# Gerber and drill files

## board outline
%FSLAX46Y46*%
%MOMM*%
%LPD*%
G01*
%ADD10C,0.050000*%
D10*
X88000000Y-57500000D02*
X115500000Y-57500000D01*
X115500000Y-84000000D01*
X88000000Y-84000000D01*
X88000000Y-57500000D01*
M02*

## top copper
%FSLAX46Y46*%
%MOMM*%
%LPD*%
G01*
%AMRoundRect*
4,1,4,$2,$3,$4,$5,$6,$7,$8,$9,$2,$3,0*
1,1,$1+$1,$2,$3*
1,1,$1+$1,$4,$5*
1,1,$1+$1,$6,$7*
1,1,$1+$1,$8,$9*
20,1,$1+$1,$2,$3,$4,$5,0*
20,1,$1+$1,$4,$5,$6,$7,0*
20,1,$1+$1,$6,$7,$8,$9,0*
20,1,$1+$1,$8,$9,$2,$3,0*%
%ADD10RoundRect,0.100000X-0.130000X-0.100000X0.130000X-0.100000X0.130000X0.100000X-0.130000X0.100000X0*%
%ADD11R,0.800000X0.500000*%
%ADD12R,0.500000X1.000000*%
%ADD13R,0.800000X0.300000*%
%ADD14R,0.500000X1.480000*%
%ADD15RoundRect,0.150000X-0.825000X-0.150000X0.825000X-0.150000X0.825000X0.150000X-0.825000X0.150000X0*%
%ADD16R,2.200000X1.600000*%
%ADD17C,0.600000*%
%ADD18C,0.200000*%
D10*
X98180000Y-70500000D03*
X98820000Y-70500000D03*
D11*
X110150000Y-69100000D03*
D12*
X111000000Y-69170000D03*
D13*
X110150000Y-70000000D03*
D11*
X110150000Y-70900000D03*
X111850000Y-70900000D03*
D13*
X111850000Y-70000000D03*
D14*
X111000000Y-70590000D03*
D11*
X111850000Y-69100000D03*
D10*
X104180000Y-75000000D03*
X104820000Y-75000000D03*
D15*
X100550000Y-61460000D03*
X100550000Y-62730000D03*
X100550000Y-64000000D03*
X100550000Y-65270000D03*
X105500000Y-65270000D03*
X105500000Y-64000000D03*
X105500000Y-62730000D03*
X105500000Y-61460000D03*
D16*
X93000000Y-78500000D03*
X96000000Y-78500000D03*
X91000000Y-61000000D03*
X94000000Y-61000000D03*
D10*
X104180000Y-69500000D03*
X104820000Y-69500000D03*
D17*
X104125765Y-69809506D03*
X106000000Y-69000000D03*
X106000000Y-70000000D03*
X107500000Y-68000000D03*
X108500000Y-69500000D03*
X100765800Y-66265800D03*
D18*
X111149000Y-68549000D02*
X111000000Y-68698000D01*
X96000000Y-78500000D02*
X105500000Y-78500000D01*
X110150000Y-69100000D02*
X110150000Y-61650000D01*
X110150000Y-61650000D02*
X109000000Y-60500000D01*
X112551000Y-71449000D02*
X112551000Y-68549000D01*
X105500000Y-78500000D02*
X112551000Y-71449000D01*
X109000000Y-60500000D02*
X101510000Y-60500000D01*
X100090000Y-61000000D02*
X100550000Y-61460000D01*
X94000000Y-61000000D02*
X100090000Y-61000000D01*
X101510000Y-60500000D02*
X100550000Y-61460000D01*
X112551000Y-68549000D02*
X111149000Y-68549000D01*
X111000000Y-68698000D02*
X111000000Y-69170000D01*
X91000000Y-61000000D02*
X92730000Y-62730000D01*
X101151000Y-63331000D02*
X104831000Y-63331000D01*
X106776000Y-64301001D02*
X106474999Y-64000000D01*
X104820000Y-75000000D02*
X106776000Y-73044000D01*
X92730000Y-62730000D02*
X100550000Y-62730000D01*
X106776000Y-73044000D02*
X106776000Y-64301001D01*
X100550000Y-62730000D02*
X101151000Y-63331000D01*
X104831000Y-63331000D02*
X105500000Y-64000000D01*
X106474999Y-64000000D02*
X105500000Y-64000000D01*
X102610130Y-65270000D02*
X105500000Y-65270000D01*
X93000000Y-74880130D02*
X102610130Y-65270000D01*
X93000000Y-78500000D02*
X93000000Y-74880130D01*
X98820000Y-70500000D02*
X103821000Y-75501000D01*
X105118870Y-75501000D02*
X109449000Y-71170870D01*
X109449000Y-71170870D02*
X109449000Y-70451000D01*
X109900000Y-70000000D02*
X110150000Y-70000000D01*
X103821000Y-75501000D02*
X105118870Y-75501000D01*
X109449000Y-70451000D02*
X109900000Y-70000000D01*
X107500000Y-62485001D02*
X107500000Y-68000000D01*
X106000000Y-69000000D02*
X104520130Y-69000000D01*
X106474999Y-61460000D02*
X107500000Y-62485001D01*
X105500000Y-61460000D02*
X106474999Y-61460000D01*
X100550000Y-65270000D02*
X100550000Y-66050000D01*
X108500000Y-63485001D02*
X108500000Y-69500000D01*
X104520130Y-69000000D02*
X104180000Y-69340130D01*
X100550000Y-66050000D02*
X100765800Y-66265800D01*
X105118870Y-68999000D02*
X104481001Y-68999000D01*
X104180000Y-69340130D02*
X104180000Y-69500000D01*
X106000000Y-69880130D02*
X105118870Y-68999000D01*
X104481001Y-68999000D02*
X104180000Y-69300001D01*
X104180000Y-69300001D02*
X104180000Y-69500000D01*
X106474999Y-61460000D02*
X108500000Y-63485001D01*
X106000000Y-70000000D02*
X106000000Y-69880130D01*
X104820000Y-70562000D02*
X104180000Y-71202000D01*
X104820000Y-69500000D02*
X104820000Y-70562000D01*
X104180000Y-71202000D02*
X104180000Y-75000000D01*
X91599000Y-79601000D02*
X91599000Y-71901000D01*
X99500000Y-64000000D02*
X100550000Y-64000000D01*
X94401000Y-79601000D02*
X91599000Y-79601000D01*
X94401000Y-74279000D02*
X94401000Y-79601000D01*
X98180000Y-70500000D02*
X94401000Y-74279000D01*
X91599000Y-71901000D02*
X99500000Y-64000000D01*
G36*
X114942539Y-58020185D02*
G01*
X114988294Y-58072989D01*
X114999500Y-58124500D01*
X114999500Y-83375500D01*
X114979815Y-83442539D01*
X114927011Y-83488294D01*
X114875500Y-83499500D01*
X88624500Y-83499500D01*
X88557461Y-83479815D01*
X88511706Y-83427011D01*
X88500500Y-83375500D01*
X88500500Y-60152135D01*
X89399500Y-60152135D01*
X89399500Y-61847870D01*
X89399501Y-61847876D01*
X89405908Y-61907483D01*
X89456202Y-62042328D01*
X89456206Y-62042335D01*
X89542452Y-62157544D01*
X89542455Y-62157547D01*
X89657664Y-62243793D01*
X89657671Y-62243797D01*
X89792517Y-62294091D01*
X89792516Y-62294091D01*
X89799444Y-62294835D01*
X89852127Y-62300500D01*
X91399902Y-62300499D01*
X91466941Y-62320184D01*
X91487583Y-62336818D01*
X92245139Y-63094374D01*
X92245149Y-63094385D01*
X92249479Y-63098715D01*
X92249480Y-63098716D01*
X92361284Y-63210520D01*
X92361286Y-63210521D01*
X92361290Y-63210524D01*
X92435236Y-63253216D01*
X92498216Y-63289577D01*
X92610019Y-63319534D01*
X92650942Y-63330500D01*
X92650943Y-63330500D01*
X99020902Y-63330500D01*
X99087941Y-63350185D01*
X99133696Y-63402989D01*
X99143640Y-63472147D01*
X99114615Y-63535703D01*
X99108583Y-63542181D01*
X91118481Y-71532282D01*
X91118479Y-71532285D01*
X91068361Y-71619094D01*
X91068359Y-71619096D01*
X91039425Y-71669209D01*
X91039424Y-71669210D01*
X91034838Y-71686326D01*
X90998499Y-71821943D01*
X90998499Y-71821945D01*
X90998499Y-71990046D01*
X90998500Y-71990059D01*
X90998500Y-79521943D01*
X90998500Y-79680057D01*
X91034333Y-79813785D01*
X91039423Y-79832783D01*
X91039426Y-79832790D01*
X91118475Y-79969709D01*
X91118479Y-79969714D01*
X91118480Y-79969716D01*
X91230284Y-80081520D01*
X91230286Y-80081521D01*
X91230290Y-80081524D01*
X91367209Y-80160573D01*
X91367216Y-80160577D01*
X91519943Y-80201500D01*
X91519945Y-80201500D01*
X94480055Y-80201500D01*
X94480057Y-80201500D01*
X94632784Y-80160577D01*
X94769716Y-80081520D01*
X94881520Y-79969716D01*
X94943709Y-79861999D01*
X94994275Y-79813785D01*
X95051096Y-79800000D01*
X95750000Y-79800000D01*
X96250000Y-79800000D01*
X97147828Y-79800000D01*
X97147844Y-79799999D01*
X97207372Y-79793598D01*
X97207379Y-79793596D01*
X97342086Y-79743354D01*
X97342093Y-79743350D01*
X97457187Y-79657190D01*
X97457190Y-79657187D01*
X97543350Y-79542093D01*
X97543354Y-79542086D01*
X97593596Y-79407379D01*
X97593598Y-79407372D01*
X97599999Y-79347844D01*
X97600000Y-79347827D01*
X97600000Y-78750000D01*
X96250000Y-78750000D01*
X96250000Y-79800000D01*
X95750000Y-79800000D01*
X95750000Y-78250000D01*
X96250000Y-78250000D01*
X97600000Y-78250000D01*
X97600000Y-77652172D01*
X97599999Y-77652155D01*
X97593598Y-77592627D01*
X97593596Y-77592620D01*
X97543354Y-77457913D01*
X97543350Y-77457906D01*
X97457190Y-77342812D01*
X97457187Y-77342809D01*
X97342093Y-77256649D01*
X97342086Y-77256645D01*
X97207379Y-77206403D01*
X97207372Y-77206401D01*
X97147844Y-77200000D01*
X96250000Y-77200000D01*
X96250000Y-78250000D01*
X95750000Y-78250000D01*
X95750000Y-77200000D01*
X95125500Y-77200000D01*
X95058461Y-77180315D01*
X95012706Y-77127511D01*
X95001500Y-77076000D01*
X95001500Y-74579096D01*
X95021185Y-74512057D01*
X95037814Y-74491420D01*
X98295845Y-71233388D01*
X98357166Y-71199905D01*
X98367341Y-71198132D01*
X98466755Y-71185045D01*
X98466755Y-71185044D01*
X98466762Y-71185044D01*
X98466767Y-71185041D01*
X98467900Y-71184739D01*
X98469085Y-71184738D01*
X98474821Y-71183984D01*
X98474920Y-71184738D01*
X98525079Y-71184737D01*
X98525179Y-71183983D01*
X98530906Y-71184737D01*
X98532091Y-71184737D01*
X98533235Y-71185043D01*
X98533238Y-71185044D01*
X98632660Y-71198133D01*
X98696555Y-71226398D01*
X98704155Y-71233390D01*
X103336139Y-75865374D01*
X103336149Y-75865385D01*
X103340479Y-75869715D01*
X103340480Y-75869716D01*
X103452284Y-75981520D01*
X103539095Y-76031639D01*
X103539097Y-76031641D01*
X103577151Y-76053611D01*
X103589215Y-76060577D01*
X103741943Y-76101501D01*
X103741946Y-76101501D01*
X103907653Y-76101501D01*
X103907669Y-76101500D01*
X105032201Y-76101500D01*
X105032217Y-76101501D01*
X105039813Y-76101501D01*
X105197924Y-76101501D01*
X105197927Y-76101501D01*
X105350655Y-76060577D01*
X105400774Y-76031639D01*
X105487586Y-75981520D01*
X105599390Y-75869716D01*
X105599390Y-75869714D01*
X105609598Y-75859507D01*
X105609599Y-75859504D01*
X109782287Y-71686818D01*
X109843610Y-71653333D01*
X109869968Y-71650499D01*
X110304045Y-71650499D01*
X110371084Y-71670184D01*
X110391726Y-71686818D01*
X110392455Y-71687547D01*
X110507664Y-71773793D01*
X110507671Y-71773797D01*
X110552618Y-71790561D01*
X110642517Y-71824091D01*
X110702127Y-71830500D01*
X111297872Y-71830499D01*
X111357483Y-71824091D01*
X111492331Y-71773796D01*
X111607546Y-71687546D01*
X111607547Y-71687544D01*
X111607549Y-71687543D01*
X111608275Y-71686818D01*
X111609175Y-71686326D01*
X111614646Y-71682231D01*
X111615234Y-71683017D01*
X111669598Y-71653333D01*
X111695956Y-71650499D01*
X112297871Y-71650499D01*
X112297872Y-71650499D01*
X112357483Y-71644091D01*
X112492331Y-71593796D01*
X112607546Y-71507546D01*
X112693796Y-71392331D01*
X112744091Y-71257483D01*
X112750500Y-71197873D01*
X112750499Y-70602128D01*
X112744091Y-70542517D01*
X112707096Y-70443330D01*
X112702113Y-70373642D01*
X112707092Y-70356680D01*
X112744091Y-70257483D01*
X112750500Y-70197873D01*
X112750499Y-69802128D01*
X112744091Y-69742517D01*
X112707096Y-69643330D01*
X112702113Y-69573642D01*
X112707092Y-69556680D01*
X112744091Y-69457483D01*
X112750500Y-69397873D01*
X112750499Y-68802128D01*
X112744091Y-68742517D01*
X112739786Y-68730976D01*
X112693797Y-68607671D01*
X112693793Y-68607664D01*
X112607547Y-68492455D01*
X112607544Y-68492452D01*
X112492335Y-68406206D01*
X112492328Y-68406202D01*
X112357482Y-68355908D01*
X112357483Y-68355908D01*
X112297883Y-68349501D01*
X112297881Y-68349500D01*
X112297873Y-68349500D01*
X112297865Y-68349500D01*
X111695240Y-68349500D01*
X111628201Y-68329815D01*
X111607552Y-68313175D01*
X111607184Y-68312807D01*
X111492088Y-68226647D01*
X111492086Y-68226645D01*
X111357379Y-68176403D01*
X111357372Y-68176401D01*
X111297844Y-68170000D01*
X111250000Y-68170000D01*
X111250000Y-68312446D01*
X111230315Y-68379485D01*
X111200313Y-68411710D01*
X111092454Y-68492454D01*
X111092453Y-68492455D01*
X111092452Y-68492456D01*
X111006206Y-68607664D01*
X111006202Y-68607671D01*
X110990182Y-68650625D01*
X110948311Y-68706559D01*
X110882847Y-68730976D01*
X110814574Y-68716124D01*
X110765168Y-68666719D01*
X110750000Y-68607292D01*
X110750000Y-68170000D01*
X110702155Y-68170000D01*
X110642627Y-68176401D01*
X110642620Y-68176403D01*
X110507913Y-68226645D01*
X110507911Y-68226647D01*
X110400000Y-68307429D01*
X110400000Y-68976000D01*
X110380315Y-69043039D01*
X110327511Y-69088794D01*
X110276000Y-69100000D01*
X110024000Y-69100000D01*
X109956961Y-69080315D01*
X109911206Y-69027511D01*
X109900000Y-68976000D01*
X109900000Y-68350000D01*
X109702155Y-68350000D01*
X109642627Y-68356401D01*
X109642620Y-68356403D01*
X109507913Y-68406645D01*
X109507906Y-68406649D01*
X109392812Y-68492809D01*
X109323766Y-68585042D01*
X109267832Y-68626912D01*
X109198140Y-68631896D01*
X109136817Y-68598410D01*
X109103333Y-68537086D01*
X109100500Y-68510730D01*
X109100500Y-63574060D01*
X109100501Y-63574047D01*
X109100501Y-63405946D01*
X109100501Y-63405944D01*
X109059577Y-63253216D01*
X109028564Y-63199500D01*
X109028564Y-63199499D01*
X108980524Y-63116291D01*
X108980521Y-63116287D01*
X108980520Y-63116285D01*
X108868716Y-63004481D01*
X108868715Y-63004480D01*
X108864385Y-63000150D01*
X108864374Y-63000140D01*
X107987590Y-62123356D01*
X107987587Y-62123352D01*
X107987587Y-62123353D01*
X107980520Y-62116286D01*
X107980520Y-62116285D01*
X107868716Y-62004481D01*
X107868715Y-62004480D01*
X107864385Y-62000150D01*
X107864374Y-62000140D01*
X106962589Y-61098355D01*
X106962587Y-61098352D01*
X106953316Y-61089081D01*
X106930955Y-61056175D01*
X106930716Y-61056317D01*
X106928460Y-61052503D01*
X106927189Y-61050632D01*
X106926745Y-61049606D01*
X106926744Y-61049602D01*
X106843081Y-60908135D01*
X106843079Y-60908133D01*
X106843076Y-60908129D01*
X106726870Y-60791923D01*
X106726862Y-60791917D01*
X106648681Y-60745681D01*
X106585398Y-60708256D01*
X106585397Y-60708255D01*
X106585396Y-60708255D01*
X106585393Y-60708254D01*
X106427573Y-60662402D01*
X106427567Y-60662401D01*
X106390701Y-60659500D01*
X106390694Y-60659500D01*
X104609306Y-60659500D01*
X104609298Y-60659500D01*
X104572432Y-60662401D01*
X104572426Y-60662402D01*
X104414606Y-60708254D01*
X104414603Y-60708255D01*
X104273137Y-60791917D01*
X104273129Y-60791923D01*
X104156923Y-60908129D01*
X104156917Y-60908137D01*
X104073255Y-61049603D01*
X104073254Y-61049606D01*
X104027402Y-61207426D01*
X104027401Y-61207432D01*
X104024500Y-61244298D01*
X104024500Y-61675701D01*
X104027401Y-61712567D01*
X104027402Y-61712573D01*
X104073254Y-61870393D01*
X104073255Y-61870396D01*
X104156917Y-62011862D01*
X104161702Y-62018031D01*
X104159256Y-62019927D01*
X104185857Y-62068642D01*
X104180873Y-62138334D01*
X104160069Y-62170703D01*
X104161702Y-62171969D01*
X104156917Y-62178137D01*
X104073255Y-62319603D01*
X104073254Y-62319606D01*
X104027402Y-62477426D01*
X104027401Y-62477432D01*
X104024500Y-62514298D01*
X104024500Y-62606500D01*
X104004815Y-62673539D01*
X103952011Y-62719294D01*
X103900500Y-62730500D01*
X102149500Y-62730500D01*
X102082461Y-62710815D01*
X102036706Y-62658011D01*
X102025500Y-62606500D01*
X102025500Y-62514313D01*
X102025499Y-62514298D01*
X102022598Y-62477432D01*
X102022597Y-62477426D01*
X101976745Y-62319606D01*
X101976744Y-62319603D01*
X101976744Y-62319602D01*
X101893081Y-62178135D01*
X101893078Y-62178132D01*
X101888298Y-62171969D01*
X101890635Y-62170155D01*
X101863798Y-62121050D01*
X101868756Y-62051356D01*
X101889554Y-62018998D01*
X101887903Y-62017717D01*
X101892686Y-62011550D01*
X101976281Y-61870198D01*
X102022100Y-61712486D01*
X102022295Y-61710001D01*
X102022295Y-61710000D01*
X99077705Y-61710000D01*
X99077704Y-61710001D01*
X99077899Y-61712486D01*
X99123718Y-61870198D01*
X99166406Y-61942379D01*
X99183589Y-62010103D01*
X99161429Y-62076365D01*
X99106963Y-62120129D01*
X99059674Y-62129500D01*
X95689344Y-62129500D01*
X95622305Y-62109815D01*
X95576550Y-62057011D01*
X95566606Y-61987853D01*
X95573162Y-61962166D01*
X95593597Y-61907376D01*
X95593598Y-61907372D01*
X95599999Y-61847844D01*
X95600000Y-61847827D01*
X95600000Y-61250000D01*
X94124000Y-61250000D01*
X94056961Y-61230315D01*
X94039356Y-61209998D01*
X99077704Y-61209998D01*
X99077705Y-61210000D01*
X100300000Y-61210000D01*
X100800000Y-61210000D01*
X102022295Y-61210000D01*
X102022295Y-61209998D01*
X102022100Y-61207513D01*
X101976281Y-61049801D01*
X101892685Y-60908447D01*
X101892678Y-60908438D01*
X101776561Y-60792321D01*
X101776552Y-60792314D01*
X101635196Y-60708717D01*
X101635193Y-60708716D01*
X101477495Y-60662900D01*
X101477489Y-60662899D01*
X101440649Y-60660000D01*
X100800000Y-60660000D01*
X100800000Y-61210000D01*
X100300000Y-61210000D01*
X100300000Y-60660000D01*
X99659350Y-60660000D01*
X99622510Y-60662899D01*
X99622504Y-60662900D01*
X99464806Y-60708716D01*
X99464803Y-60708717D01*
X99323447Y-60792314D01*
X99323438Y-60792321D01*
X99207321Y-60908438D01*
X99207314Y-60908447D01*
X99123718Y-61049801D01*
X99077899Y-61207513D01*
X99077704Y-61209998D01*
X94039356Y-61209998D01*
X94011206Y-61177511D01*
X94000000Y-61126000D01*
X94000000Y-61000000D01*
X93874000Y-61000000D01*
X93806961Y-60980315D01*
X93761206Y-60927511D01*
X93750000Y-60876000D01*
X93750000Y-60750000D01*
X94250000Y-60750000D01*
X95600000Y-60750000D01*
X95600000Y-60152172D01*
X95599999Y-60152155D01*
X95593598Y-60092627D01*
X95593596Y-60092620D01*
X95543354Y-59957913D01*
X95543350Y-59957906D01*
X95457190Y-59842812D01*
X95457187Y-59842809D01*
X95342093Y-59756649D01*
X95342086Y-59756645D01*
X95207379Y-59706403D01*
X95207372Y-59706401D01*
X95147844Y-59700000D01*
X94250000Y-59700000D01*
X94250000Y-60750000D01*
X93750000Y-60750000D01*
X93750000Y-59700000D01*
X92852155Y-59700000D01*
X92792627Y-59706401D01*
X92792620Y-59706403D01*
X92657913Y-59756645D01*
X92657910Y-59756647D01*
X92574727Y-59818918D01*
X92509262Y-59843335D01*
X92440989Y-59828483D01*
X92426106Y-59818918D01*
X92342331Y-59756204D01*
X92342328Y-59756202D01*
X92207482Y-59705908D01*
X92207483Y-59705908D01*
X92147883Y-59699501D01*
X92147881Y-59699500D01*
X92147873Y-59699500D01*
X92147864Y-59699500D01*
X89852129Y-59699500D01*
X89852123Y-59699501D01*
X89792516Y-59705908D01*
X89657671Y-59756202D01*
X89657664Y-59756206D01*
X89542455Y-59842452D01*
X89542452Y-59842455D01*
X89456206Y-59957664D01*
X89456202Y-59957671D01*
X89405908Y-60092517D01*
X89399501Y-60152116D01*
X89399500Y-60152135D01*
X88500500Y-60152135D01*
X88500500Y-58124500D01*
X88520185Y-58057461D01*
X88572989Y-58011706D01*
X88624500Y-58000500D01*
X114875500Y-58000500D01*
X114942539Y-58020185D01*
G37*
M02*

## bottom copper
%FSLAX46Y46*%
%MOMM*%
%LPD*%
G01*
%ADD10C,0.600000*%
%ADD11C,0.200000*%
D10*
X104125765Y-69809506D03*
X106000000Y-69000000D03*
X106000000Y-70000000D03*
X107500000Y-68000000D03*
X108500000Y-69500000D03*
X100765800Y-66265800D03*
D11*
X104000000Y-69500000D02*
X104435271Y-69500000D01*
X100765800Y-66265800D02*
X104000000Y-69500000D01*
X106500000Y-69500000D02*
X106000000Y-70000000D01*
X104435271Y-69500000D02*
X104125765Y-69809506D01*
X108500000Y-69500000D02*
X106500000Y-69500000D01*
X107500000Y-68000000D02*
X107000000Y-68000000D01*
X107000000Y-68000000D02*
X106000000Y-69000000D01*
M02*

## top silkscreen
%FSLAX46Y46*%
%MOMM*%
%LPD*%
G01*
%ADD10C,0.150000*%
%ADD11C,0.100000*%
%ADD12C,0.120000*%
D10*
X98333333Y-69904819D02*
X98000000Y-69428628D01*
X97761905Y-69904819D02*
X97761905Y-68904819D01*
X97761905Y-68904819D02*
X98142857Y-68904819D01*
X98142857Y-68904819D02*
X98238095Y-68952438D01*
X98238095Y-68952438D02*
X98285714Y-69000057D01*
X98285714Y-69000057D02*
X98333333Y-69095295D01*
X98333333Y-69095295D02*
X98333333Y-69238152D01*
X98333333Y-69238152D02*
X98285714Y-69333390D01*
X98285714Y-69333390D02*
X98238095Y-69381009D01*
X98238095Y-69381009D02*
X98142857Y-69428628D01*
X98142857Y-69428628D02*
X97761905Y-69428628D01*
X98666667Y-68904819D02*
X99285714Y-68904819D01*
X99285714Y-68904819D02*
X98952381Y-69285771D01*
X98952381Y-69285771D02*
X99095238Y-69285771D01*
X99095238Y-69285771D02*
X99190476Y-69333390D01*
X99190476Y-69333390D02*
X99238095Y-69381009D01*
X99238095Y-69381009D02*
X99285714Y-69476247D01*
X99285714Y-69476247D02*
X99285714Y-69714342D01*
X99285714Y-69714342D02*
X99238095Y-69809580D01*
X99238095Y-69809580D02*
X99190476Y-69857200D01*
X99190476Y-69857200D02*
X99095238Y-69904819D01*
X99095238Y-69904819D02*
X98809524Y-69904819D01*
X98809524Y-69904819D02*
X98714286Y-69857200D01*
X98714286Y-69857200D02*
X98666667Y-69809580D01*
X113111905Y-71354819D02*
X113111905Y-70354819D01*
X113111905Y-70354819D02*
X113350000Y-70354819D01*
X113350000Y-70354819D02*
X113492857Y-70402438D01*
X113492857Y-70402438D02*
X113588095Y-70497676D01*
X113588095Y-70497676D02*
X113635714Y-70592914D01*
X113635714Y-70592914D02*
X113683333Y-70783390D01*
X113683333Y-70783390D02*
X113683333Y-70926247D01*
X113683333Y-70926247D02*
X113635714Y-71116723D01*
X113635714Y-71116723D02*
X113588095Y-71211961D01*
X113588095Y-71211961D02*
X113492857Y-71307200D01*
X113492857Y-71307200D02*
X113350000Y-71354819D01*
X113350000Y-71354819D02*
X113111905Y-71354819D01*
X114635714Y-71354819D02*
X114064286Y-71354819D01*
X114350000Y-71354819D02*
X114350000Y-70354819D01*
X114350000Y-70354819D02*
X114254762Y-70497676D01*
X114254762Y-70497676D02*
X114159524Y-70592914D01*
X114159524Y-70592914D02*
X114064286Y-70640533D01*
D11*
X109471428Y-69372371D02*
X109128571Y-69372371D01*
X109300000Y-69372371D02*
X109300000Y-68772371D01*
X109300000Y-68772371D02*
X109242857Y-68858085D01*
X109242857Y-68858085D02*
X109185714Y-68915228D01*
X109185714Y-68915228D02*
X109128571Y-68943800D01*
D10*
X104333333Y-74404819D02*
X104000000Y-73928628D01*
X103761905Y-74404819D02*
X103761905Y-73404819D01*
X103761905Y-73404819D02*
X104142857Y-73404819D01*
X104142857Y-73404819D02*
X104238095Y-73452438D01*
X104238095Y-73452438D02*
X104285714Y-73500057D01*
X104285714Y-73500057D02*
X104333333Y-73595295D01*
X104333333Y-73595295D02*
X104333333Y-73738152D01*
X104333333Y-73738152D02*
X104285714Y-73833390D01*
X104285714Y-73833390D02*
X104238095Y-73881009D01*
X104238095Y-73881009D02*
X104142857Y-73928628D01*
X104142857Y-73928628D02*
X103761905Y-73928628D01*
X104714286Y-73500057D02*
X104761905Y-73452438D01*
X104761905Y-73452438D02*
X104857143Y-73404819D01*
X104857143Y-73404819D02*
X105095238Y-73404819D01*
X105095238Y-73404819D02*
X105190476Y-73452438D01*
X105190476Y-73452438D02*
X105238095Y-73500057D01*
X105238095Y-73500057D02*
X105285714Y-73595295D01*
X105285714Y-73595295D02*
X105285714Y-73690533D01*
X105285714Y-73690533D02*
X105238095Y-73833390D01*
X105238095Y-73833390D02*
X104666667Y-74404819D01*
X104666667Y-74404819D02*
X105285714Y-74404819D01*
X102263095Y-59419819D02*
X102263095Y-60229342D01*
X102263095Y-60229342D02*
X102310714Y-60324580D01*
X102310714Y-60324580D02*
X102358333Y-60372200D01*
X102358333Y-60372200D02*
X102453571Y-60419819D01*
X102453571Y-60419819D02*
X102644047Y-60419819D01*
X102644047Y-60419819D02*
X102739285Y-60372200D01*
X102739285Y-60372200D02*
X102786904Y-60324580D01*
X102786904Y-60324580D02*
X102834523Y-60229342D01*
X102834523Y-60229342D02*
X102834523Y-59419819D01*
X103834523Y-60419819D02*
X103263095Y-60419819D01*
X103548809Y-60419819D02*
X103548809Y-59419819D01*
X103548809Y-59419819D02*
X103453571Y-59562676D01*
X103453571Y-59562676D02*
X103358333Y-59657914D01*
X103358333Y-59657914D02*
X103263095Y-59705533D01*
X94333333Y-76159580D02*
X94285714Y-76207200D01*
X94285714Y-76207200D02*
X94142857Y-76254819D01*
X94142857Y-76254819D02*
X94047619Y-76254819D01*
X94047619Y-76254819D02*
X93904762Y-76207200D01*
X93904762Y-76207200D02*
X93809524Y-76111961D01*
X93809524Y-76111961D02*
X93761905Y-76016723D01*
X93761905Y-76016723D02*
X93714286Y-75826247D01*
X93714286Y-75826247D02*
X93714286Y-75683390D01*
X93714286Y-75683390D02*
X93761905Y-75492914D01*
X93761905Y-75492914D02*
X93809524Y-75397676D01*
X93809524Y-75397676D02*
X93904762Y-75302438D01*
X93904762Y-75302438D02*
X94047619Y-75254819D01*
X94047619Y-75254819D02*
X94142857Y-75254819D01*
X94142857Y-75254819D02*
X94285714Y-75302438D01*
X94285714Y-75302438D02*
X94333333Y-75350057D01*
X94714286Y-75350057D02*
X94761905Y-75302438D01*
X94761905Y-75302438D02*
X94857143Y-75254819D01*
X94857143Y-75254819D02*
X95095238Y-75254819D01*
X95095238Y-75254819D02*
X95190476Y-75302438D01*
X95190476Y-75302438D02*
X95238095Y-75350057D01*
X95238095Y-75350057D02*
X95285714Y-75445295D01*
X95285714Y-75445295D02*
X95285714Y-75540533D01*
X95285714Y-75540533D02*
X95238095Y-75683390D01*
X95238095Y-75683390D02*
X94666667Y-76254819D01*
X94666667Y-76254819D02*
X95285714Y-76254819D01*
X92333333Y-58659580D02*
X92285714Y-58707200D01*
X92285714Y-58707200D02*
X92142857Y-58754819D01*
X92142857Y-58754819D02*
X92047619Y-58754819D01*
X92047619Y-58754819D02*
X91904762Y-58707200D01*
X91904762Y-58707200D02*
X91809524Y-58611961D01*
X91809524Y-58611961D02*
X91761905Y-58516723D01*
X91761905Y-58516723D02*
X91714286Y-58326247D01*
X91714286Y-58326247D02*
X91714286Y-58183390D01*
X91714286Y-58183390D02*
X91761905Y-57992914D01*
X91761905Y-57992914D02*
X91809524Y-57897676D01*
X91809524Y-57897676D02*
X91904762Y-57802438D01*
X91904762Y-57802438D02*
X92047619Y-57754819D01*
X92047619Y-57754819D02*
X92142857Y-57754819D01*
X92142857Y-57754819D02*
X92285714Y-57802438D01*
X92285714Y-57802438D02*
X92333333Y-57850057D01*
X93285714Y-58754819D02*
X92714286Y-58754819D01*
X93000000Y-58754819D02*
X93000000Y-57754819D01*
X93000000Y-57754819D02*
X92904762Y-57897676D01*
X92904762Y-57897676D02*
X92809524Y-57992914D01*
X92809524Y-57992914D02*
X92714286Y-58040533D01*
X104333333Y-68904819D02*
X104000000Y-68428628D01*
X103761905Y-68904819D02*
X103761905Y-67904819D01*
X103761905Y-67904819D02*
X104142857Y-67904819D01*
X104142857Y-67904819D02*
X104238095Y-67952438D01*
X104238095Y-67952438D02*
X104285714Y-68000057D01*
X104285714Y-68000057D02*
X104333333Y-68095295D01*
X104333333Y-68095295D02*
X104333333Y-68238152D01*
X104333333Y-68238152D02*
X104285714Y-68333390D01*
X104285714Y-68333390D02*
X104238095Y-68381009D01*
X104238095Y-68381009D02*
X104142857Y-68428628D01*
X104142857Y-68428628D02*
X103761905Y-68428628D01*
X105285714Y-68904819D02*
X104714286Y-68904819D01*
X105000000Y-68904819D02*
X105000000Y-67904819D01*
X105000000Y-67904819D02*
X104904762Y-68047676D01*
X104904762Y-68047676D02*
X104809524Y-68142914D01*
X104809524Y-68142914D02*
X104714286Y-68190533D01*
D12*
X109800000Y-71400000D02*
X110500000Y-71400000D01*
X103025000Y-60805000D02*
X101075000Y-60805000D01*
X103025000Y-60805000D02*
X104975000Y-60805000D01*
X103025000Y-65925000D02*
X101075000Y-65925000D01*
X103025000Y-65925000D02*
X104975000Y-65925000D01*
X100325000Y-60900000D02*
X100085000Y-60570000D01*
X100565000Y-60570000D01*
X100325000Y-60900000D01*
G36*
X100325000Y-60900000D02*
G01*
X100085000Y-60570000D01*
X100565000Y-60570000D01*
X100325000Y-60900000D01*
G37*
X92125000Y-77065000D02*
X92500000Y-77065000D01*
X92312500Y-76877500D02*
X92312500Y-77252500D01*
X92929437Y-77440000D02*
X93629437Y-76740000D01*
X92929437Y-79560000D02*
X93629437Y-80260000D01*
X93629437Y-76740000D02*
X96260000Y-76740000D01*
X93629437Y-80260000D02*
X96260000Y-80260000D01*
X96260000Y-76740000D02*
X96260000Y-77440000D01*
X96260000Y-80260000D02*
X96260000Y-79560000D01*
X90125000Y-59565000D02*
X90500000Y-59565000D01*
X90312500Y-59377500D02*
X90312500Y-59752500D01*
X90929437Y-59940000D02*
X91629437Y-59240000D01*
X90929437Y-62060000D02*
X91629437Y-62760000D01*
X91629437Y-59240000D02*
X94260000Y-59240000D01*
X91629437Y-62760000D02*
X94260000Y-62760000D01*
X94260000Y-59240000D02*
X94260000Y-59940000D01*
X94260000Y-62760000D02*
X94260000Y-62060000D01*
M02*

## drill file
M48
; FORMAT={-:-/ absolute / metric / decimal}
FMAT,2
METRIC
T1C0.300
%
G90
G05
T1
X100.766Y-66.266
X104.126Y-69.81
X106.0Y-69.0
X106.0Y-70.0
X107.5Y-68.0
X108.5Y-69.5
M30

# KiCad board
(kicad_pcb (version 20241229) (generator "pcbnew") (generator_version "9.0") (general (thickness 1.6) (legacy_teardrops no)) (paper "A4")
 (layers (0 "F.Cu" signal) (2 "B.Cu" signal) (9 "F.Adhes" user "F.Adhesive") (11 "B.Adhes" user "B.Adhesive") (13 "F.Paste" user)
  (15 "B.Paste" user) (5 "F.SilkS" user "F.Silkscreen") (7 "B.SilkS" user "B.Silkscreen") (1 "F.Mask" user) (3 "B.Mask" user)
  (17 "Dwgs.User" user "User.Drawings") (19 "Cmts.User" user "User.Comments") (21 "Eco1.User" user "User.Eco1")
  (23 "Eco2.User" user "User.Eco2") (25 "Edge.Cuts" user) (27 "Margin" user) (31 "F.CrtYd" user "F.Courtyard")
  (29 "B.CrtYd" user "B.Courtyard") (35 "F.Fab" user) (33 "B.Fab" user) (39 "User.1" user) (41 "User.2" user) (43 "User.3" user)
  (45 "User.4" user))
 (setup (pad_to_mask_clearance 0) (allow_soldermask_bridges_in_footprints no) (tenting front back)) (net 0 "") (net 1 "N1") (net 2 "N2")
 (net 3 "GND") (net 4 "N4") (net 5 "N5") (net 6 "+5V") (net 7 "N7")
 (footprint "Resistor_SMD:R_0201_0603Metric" (layer "F.Cu") (at 98.5 70.5)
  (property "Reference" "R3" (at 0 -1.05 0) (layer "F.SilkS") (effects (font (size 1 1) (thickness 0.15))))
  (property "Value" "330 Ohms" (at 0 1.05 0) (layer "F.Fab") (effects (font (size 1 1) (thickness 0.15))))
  (pad "" smd roundrect (at -0.345 0) (size 0.318 0.36) (layers "F.Paste") (roundrect_rratio 0.25))
  (pad "" smd roundrect (at 0.345 0) (size 0.318 0.36) (layers "F.Paste") (roundrect_rratio 0.25))
  (pad "1" smd roundrect (at -0.32 0) (size 0.46 0.4) (layers "F.Cu" "F.Mask") (roundrect_rratio 0.25) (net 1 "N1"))
  (pad "2" smd roundrect (at 0.32 0) (size 0.46 0.4) (layers "F.Cu" "F.Mask") (roundrect_rratio 0.25) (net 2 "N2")))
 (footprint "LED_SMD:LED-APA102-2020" (layer "F.Cu") (at 111 70)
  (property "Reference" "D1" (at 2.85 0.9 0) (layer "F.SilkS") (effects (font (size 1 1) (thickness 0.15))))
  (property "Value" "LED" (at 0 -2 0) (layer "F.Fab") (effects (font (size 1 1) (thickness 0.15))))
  (fp_line (start -1.2 1.4) (end -0.5 1.4) (stroke (width 0.12) (type solid)) (layer "F.SilkS"))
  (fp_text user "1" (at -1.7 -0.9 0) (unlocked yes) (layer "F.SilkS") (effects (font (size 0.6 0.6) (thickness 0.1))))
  (pad "1" smd rect (at -0.85 -0.9) (size 0.8 0.5) (layers "F.Cu" "F.Mask" "F.Paste") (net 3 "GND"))
  (pad "1" smd rect (at 0 -0.83 90) (size 1 0.5) (layers "F.Cu" "F.Mask" "F.Paste") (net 3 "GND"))
  (pad "2" smd rect (at -0.85 0) (size 0.8 0.3) (layers "F.Cu" "F.Mask" "F.Paste") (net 2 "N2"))
  (pad "3" smd rect (at -0.85 0.9) (size 0.8 0.5) (layers "F.Cu" "F.Mask" "F.Paste"))
  (pad "4" smd rect (at 0.85 0.9) (size 0.8 0.5) (layers "F.Cu" "F.Mask" "F.Paste"))
  (pad "5" smd rect (at 0.85 0) (size 0.8 0.3) (layers "F.Cu" "F.Mask" "F.Paste"))
  (pad "6" smd rect (at 0 0.59 90) (size 1.48 0.5) (layers "F.Cu" "F.Mask" "F.Paste"))
  (pad "6" smd rect (at 0.85 -0.9) (size 0.8 0.5) (layers "F.Cu" "F.Mask" "F.Paste")))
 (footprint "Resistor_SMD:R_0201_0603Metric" (layer "F.Cu") (at 104.5 75)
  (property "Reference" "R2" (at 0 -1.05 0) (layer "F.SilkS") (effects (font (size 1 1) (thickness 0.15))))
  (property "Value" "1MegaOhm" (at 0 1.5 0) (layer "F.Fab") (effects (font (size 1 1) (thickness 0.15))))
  (pad "" smd roundrect (at -0.345 0) (size 0.318 0.36) (layers "F.Paste") (roundrect_rratio 0.25))
  (pad "" smd roundrect (at 0.345 0) (size 0.318 0.36) (layers "F.Paste") (roundrect_rratio 0.25))
  (pad "1" smd roundrect (at -0.32 0) (size 0.46 0.4) (layers "F.Cu" "F.Mask") (roundrect_rratio 0.25) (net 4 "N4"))
  (pad "2" smd roundrect (at 0.32 0) (size 0.46 0.4) (layers "F.Cu" "F.Mask") (roundrect_rratio 0.25) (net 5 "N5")))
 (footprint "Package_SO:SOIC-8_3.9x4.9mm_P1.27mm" (layer "F.Cu") (at 103.025 63.365)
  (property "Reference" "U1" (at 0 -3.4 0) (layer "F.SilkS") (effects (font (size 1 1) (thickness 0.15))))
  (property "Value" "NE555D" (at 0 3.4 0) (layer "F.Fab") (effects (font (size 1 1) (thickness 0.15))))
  (fp_line (start 0 -2.56) (end -1.95 -2.56) (stroke (width 0.12) (type solid)) (layer "F.SilkS"))
  (fp_line (start 0 -2.56) (end 1.95 -2.56) (stroke (width 0.12) (type solid)) (layer "F.SilkS"))
  (fp_line (start 0 2.56) (end -1.95 2.56) (stroke (width 0.12) (type solid)) (layer "F.SilkS"))
  (fp_line (start 0 2.56) (end 1.95 2.56) (stroke (width 0.12) (type solid)) (layer "F.SilkS"))
  (fp_poly (pts (xy -2.7 -2.465) (xy -2.94 -2.795) (xy -2.46 -2.795)) (stroke (width 0.12) (type solid)) (fill yes) (layer "F.SilkS"))
  (pad "1" smd roundrect (at -2.475 -1.905) (size 1.95 0.6) (layers "F.Cu" "F.Mask" "F.Paste") (roundrect_rratio 0.25) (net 3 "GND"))
  (pad "2" smd roundrect (at -2.475 -0.635) (size 1.95 0.6) (layers "F.Cu" "F.Mask" "F.Paste") (roundrect_rratio 0.25) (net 5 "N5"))
  (pad "3" smd roundrect (at -2.475 0.635) (size 1.95 0.6) (layers "F.Cu" "F.Mask" "F.Paste") (roundrect_rratio 0.25) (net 1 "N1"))
  (pad "4" smd roundrect (at -2.475 1.905) (size 1.95 0.6) (layers "F.Cu" "F.Mask" "F.Paste") (roundrect_rratio 0.25) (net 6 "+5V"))
  (pad "5" smd roundrect (at 2.475 1.905) (size 1.95 0.6) (layers "F.Cu" "F.Mask" "F.Paste") (roundrect_rratio 0.25) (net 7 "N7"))
  (pad "6" smd roundrect (at 2.475 0.635) (size 1.95 0.6) (layers "F.Cu" "F.Mask" "F.Paste") (roundrect_rratio 0.25) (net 5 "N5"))
  (pad "7" smd roundrect (at 2.475 -0.635) (size 1.95 0.6) (layers "F.Cu" "F.Mask" "F.Paste") (roundrect_rratio 0.25) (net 4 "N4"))
  (pad "8" smd roundrect (at 2.475 -1.905) (size 1.95 0.6) (layers "F.Cu" "F.Mask" "F.Paste") (roundrect_rratio 0.25) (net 6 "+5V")))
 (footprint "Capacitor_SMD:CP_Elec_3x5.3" (layer "F.Cu") (at 94.5 78.5)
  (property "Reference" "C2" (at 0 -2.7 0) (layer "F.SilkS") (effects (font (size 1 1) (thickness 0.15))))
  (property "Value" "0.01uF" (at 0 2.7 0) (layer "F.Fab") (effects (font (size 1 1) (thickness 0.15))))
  (fp_line (start -2.375 -1.435) (end -2 -1.435) (stroke (width 0.12) (type solid)) (layer "F.SilkS"))
  (fp_line (start -2.1875 -1.6225) (end -2.1875 -1.2475) (stroke (width 0.12) (type solid)) (layer "F.SilkS"))
  (fp_line (start -1.570563 -1.06) (end -0.870563 -1.76) (stroke (width 0.12) (type solid)) (layer "F.SilkS"))
  (fp_line (start -1.570563 1.06) (end -0.870563 1.76) (stroke (width 0.12) (type solid)) (layer "F.SilkS"))
  (fp_line (start -0.870563 -1.76) (end 1.76 -1.76) (stroke (width 0.12) (type solid)) (layer "F.SilkS"))
  (fp_line (start -0.870563 1.76) (end 1.76 1.76) (stroke (width 0.12) (type solid)) (layer "F.SilkS"))
  (fp_line (start 1.76 -1.76) (end 1.76 -1.06) (stroke (width 0.12) (type solid)) (layer "F.SilkS"))
  (fp_line (start 1.76 1.76) (end 1.76 1.06) (stroke (width 0.12) (type solid)) (layer "F.SilkS"))
  (pad "1" smd rect (at -1.5 0) (size 2.2 1.6) (layers "F.Cu" "F.Mask" "F.Paste") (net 7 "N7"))
  (pad "2" smd rect (at 1.5 0) (size 2.2 1.6) (layers "F.Cu" "F.Mask" "F.Paste") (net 3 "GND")))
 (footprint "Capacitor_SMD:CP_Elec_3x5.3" (layer "F.Cu") (at 92.5 61)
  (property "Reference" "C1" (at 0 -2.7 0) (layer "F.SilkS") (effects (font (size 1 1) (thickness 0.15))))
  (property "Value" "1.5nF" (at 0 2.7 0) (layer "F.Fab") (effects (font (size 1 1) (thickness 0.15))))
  (fp_line (start -2.375 -1.435) (end -2 -1.435) (stroke (width 0.12) (type solid)) (layer "F.SilkS"))
  (fp_line (start -2.1875 -1.6225) (end -2.1875 -1.2475) (stroke (width 0.12) (type solid)) (layer "F.SilkS"))
  (fp_line (start -1.570563 -1.06) (end -0.870563 -1.76) (stroke (width 0.12) (type solid)) (layer "F.SilkS"))
  (fp_line (start -1.570563 1.06) (end -0.870563 1.76) (stroke (width 0.12) (type solid)) (layer "F.SilkS"))
  (fp_line (start -0.870563 -1.76) (end 1.76 -1.76) (stroke (width 0.12) (type solid)) (layer "F.SilkS"))
  (fp_line (start -0.870563 1.76) (end 1.76 1.76) (stroke (width 0.12) (type solid)) (layer "F.SilkS"))
  (fp_line (start 1.76 -1.76) (end 1.76 -1.06) (stroke (width 0.12) (type solid)) (layer "F.SilkS"))
  (fp_line (start 1.76 1.76) (end 1.76 1.06) (stroke (width 0.12) (type solid)) (layer "F.SilkS"))
  (pad "1" smd rect (at -1.5 0) (size 2.2 1.6) (layers "F.Cu" "F.Mask" "F.Paste") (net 5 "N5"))
  (pad "2" smd rect (at 1.5 0) (size 2.2 1.6) (layers "F.Cu" "F.Mask" "F.Paste") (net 3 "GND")))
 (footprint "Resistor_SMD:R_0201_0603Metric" (layer "F.Cu") (at 104.5 69.5)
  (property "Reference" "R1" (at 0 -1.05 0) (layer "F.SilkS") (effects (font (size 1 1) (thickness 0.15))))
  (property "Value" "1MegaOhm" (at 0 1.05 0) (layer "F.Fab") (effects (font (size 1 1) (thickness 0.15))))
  (pad "" smd roundrect (at -0.345 0) (size 0.318 0.36) (layers "F.Paste") (roundrect_rratio 0.25))
  (pad "" smd roundrect (at 0.345 0) (size 0.318 0.36) (layers "F.Paste") (roundrect_rratio 0.25))
  (pad "1" smd roundrect (at -0.32 0) (size 0.46 0.4) (layers "F.Cu" "F.Mask") (roundrect_rratio 0.25) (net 6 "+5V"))
  (pad "2" smd roundrect (at 0.32 0) (size 0.46 0.4) (layers "F.Cu" "F.Mask") (roundrect_rratio 0.25) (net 4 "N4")))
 (gr_rect (start 88 57.5) (end 115.5 84) (stroke (width 0.05) (type default)) (fill no) (layer "Edge.Cuts"))
 (segment (start 111.149 68.549) (end 111 68.698) (width 0.2) (layer "F.Cu") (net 3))
 (segment (start 96 78.5) (end 105.5 78.5) (width 0.2) (layer "F.Cu") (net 3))
 (segment (start 110.15 69.1) (end 110.15 61.65) (width 0.2) (layer "F.Cu") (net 3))
 (segment (start 110.15 61.65) (end 109 60.5) (width 0.2) (layer "F.Cu") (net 3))
 (segment (start 112.551 71.449) (end 112.551 68.549) (width 0.2) (layer "F.Cu") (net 3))
 (segment (start 105.5 78.5) (end 112.551 71.449) (width 0.2) (layer "F.Cu") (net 3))
 (segment (start 109 60.5) (end 101.51 60.5) (width 0.2) (layer "F.Cu") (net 3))
 (segment (start 100.09 61) (end 100.55 61.46) (width 0.2) (layer "F.Cu") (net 3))
 (segment (start 94 61) (end 100.09 61) (width 0.2) (layer "F.Cu") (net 3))
 (segment (start 101.51 60.5) (end 100.55 61.46) (width 0.2) (layer "F.Cu") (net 3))
 (segment (start 112.551 68.549) (end 111.149 68.549) (width 0.2) (layer "F.Cu") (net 3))
 (segment (start 111 68.698) (end 111 69.17) (width 0.2) (layer "F.Cu") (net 3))
 (segment (start 91 61) (end 92.73 62.73) (width 0.2) (layer "F.Cu") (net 5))
 (segment (start 101.151 63.331) (end 104.831 63.331) (width 0.2) (layer "F.Cu") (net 5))
 (segment (start 106.776 64.301001) (end 106.474999 64) (width 0.2) (layer "F.Cu") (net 5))
 (segment (start 104.82 75) (end 106.776 73.044) (width 0.2) (layer "F.Cu") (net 5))
 (segment (start 92.73 62.73) (end 100.55 62.73) (width 0.2) (layer "F.Cu") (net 5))
 (segment (start 106.776 73.044) (end 106.776 64.301001) (width 0.2) (layer "F.Cu") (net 5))
 (segment (start 100.55 62.73) (end 101.151 63.331) (width 0.2) (layer "F.Cu") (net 5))
 (segment (start 104.831 63.331) (end 105.5 64) (width 0.2) (layer "F.Cu") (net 5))
 (segment (start 106.474999 64) (end 105.5 64) (width 0.2) (layer "F.Cu") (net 5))
 (segment (start 102.61013 65.27) (end 105.5 65.27) (width 0.2) (layer "F.Cu") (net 7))
 (segment (start 93 74.88013) (end 102.61013 65.27) (width 0.2) (layer "F.Cu") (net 7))
 (segment (start 93 78.5) (end 93 74.88013) (width 0.2) (layer "F.Cu") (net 7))
 (segment (start 98.82 70.5) (end 103.821 75.501) (width 0.2) (layer "F.Cu") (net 2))
 (segment (start 105.11887 75.501) (end 109.449 71.17087) (width 0.2) (layer "F.Cu") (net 2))
 (segment (start 109.449 71.17087) (end 109.449 70.451) (width 0.2) (layer "F.Cu") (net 2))
 (segment (start 109.9 70) (end 110.15 70) (width 0.2) (layer "F.Cu") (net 2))
 (segment (start 103.821 75.501) (end 105.11887 75.501) (width 0.2) (layer "F.Cu") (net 2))
 (segment (start 109.449 70.451) (end 109.9 70) (width 0.2) (layer "F.Cu") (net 2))
 (segment (start 107.5 62.485001) (end 107.5 68) (width 0.2) (layer "F.Cu") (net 6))
 (segment (start 106 69) (end 104.52013 69) (width 0.2) (layer "F.Cu") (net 6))
 (segment (start 106.474999 61.46) (end 107.5 62.485001) (width 0.2) (layer "F.Cu") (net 6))
 (segment (start 105.5 61.46) (end 106.474999 61.46) (width 0.2) (layer "F.Cu") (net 6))
 (segment (start 100.55 65.27) (end 100.55 66.05) (width 0.2) (layer "F.Cu") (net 6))
 (segment (start 108.5 63.485001) (end 108.5 69.5) (width 0.2) (layer "F.Cu") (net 6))
 (segment (start 104.52013 69) (end 104.18 69.34013) (width 0.2) (layer "F.Cu") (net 6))
 (segment (start 100.55 66.05) (end 100.7658 66.2658) (width 0.2) (layer "F.Cu") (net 6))
 (segment (start 105.11887 68.999) (end 104.481001 68.999) (width 0.2) (layer "F.Cu") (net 6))
 (segment (start 104.18 69.34013) (end 104.18 69.5) (width 0.2) (layer "F.Cu") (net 6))
 (segment (start 106 69.88013) (end 105.11887 68.999) (width 0.2) (layer "F.Cu") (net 6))
 (segment (start 104.481001 68.999) (end 104.18 69.300001) (width 0.2) (layer "F.Cu") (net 6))
 (segment (start 104.18 69.300001) (end 104.18 69.5) (width 0.2) (layer "F.Cu") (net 6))
 (segment (start 106.474999 61.46) (end 108.5 63.485001) (width 0.2) (layer "F.Cu") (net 6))
 (segment (start 106 70) (end 106 69.88013) (width 0.2) (layer "F.Cu") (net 6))
 (via (at 104.125765 69.809506) (size 0.6) (drill 0.3) (layers "F.Cu" "B.Cu") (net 6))
 (via (at 106 69) (size 0.6) (drill 0.3) (layers "F.Cu" "B.Cu") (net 6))
 (via (at 106 70) (size 0.6) (drill 0.3) (layers "F.Cu" "B.Cu") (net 6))
 (via (at 107.5 68) (size 0.6) (drill 0.3) (layers "F.Cu" "B.Cu") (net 6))
 (via (at 108.5 69.5) (size 0.6) (drill 0.3) (layers "F.Cu" "B.Cu") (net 6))
 (via (at 100.7658 66.2658) (size 0.6) (drill 0.3) (layers "F.Cu" "B.Cu") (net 6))
 (segment (start 104 69.5) (end 104.435271 69.5) (width 0.2) (layer "B.Cu") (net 6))
 (segment (start 100.7658 66.2658) (end 104 69.5) (width 0.2) (layer "B.Cu") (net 6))
 (segment (start 106.5 69.5) (end 106 70) (width 0.2) (layer "B.Cu") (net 6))
 (segment (start 104.435271 69.5) (end 104.125765 69.809506) (width 0.2) (layer "B.Cu") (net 6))
 (segment (start 108.5 69.5) (end 106.5 69.5) (width 0.2) (layer "B.Cu") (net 6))
 (segment (start 107.5 68) (end 107 68) (width 0.2) (layer "B.Cu") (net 6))
 (segment (start 107 68) (end 106 69) (width 0.2) (layer "B.Cu") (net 6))
 (segment (start 104.82 70.562) (end 104.18 71.202) (width 0.2) (layer "F.Cu") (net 4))
 (segment (start 104.82 69.5) (end 104.82 70.562) (width 0.2) (layer "F.Cu") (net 4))
 (segment (start 104.18 71.202) (end 104.18 75) (width 0.2) (layer "F.Cu") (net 4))
 (segment (start 91.599 79.601) (end 91.599 71.901) (width 0.2) (layer "F.Cu") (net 1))
 (segment (start 99.5 64) (end 100.55 64) (width 0.2) (layer "F.Cu") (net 1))
 (segment (start 94.401 79.601) (end 91.599 79.601) (width 0.2) (layer "F.Cu") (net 1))
 (segment (start 94.401 74.279) (end 94.401 79.601) (width 0.2) (layer "F.Cu") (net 1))
 (segment (start 98.18 70.5) (end 94.401 74.279) (width 0.2) (layer "F.Cu") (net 1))
 (segment (start 91.599 71.901) (end 99.5 64) (width 0.2) (layer "F.Cu") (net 1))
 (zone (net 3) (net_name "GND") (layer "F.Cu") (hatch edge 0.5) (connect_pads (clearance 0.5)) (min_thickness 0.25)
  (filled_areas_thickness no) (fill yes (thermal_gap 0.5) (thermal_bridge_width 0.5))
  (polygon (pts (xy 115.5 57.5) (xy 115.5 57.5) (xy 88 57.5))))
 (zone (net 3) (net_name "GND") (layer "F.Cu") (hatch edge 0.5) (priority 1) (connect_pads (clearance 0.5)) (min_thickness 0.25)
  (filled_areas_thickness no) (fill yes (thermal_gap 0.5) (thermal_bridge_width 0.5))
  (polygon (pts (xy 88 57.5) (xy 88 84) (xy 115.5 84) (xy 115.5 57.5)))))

